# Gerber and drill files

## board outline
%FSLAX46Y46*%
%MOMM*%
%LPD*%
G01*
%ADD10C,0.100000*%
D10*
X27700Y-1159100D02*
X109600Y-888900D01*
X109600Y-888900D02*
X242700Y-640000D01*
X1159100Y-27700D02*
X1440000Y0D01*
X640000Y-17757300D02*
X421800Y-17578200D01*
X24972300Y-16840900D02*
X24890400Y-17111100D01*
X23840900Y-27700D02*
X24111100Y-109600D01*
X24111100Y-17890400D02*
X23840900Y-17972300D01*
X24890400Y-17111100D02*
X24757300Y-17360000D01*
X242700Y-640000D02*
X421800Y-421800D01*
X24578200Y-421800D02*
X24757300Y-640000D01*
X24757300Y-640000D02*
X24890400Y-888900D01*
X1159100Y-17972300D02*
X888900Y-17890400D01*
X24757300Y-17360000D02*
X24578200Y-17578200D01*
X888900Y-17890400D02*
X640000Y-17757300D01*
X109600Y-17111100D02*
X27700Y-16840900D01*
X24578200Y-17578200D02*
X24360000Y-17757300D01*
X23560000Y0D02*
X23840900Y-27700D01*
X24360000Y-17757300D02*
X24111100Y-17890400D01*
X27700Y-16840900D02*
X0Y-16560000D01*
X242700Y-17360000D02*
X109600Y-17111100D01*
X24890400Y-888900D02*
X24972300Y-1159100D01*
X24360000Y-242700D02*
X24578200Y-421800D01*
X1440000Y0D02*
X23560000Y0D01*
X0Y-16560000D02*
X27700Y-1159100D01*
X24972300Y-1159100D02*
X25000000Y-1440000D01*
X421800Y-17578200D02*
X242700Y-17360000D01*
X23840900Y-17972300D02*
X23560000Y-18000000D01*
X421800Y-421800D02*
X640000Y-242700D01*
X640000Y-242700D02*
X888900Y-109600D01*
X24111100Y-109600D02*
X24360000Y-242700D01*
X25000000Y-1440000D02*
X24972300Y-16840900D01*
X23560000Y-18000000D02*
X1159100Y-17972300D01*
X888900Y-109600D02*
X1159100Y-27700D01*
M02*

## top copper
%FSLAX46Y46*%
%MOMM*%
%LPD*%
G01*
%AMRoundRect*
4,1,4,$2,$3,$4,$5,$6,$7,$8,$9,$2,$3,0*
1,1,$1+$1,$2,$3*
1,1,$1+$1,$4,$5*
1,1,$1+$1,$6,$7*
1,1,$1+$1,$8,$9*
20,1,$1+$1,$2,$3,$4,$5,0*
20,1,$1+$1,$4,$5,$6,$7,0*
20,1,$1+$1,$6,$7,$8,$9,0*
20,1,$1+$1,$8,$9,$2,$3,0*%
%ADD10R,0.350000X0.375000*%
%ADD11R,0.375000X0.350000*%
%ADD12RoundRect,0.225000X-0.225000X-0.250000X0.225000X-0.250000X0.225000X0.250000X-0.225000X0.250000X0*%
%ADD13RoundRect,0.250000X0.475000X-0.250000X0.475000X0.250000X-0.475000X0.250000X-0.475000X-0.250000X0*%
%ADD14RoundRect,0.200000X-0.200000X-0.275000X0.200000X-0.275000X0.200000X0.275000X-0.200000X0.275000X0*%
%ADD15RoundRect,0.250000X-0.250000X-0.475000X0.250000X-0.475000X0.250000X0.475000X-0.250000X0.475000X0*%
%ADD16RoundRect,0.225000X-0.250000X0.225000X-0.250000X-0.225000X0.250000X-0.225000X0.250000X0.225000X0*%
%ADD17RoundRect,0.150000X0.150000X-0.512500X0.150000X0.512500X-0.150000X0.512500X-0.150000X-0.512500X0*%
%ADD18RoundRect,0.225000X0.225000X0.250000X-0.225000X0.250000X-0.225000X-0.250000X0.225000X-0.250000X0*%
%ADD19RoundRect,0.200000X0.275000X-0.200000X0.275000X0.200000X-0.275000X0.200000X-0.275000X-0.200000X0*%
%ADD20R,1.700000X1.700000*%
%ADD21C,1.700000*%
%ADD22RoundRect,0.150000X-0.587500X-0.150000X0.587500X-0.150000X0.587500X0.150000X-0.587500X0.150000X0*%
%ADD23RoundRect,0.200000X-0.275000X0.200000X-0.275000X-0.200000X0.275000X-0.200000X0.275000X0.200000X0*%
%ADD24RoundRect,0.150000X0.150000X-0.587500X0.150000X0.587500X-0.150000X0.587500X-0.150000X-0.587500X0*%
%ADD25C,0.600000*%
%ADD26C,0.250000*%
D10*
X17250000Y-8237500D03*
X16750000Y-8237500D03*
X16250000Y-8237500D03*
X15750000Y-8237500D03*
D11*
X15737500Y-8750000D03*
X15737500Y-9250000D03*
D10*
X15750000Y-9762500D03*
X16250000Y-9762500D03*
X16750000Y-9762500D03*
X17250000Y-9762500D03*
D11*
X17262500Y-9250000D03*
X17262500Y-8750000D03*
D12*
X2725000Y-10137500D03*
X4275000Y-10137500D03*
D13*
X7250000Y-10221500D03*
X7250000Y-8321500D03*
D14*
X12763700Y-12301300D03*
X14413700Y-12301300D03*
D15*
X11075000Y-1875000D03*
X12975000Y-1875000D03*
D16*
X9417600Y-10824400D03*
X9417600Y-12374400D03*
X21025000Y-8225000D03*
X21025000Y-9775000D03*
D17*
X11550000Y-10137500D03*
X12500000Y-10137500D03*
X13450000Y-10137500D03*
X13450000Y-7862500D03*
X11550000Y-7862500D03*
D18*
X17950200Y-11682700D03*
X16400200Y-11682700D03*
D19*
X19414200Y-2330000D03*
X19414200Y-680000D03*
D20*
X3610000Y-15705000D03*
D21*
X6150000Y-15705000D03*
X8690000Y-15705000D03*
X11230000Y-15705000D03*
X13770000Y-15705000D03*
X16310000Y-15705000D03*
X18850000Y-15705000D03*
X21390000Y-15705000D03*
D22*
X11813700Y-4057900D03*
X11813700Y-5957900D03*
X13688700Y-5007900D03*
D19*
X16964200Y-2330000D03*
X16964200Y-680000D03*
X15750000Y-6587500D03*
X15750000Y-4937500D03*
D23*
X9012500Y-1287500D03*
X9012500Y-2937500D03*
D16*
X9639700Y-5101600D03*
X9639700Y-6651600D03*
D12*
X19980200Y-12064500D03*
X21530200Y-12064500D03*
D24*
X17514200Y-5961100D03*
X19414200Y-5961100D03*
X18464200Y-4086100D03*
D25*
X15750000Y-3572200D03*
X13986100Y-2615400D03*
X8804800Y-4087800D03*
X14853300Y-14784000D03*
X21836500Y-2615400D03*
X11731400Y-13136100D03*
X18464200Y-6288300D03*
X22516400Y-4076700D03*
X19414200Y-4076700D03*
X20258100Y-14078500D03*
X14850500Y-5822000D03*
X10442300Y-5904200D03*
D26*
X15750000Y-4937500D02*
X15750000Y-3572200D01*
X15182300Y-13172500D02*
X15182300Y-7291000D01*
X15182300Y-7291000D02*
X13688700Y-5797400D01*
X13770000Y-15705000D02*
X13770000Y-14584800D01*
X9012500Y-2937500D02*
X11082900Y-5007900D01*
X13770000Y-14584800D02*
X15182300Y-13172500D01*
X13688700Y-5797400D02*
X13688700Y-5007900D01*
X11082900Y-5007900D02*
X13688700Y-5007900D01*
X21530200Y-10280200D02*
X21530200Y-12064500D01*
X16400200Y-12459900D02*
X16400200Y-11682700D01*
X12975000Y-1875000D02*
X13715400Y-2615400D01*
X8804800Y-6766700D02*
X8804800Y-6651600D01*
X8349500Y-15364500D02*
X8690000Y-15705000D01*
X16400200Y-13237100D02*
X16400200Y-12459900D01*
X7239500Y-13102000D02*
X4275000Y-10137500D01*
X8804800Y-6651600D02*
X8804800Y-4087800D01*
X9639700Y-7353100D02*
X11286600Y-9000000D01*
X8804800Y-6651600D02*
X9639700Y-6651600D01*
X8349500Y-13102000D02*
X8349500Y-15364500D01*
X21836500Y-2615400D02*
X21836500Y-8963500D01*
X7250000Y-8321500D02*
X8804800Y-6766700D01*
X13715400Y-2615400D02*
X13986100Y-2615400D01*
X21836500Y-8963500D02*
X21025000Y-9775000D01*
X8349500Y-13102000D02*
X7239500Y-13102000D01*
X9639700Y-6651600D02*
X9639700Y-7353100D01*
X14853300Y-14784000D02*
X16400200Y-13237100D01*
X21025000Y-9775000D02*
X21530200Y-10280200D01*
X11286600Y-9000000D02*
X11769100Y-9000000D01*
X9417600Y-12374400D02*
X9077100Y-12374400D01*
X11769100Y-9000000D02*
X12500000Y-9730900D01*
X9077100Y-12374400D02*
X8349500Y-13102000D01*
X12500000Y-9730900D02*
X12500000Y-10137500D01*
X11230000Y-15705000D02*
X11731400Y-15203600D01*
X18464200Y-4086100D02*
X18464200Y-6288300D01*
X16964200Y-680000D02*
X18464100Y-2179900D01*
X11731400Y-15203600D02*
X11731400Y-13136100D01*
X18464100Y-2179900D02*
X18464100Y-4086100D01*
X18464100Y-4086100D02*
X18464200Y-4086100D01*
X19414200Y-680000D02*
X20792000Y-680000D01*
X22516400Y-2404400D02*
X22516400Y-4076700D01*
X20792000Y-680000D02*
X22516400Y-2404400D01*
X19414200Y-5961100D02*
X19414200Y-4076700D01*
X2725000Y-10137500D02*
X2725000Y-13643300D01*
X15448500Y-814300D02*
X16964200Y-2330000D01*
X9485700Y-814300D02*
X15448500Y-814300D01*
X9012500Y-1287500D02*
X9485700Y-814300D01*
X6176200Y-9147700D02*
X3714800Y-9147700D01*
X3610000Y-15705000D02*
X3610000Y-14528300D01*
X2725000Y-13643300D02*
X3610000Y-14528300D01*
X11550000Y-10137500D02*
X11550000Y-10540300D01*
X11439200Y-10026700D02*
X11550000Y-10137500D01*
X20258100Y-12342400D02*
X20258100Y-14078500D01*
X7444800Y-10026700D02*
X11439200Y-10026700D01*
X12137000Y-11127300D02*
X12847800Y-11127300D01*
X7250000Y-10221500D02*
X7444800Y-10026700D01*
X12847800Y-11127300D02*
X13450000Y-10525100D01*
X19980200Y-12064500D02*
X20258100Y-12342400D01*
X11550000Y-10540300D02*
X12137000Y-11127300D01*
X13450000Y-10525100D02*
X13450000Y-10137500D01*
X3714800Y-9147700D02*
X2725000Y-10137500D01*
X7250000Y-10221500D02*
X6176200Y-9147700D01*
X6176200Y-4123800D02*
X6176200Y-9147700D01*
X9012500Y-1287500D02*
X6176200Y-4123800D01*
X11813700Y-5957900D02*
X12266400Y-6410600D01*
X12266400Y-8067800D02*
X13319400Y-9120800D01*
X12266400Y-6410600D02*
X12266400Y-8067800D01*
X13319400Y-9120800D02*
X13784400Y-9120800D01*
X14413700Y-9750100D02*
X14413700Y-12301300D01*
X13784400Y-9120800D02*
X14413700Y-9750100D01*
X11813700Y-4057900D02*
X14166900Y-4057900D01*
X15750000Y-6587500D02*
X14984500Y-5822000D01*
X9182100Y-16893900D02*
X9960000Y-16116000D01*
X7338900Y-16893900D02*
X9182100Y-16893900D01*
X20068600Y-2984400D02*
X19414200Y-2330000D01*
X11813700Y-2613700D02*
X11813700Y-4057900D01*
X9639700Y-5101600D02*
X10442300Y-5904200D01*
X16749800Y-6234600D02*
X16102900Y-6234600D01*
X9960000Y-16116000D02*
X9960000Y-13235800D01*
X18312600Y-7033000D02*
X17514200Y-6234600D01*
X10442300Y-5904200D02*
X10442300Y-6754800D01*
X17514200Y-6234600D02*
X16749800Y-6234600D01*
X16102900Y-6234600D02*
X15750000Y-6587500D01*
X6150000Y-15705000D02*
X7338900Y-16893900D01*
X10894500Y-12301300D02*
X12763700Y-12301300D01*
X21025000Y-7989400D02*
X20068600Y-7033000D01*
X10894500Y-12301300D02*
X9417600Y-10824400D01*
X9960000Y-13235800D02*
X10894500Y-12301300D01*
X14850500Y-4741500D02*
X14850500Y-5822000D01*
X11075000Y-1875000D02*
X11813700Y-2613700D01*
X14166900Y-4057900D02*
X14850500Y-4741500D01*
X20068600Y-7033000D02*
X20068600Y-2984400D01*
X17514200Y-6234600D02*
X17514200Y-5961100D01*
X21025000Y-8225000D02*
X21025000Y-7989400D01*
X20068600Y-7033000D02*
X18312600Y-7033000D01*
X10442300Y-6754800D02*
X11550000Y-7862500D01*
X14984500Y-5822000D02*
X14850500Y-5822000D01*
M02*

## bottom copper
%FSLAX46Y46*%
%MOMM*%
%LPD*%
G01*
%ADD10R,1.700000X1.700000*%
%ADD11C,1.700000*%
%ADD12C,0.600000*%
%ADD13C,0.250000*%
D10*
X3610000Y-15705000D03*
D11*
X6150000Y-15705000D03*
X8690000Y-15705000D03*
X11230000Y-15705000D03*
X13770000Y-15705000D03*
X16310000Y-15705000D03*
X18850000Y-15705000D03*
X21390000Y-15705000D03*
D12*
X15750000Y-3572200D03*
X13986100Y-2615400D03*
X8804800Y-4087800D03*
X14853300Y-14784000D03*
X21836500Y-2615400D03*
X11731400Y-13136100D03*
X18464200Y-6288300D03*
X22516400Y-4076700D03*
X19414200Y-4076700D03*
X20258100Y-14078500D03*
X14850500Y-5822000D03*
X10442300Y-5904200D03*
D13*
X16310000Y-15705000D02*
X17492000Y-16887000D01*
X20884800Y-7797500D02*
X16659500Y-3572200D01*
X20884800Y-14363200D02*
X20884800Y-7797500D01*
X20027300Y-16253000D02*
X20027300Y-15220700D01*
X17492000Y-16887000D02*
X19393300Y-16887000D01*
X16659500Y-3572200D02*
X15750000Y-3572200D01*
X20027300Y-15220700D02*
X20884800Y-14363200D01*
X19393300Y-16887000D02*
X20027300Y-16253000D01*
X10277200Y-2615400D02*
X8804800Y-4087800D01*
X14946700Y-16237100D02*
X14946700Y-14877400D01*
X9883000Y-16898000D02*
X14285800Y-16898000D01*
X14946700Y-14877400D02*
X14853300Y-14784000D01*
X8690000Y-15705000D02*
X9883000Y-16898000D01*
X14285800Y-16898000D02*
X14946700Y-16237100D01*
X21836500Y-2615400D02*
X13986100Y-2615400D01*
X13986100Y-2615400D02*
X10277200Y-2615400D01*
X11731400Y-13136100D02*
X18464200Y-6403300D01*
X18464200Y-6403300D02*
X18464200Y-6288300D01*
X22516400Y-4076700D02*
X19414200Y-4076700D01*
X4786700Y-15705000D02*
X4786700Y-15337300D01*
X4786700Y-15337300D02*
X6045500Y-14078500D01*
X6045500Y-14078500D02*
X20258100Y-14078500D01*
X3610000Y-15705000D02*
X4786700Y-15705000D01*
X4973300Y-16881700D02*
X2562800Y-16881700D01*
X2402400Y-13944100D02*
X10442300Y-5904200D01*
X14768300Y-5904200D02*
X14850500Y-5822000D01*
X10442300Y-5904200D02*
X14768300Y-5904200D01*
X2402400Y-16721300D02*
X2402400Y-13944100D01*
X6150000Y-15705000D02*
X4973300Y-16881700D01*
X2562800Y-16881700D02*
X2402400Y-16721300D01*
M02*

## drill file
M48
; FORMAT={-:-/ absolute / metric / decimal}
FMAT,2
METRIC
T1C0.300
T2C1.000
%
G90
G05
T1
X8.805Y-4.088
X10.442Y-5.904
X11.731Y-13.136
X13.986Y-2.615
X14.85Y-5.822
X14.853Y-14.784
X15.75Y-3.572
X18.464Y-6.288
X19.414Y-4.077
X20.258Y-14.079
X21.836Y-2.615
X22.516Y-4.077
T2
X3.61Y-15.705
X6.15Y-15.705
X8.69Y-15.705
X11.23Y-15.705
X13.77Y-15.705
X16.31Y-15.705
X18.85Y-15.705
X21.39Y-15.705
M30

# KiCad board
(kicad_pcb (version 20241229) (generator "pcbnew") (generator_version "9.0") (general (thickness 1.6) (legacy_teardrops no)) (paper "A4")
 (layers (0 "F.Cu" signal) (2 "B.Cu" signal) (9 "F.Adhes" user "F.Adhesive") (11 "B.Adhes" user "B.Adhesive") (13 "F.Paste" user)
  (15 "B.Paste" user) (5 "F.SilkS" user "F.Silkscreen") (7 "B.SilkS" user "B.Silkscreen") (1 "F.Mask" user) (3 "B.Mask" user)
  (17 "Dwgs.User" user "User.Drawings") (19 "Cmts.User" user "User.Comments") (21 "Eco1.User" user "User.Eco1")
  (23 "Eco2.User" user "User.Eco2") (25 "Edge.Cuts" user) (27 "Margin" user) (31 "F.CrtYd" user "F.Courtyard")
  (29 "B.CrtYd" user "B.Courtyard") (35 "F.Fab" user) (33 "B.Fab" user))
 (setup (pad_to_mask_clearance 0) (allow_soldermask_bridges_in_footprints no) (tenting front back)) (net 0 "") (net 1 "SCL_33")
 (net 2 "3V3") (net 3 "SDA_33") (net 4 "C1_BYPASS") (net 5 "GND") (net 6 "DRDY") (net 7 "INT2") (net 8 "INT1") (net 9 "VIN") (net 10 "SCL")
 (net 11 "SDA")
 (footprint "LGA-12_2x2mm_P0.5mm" (layer "F.Cu") (at 16.5 9 -90)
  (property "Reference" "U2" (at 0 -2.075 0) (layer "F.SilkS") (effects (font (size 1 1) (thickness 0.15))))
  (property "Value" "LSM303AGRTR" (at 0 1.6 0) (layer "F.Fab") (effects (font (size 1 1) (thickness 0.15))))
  (pad "1" smd rect (at -0.7625 -0.75 270) (size 0.375 0.35) (layers "F.Cu" "F.Mask" "F.Paste") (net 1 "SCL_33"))
  (pad "2" smd rect (at -0.7625 -0.25 270) (size 0.375 0.35) (layers "F.Cu" "F.Mask" "F.Paste") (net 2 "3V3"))
  (pad "3" smd rect (at -0.7625 0.25 270) (size 0.375 0.35) (layers "F.Cu" "F.Mask" "F.Paste") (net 2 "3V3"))
  (pad "4" smd rect (at -0.7625 0.75 270) (size 0.375 0.35) (layers "F.Cu" "F.Mask" "F.Paste") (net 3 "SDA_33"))
  (pad "5" smd rect (at -0.25 0.7625) (size 0.375 0.35) (layers "F.Cu" "F.Mask" "F.Paste") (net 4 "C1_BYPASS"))
  (pad "6" smd rect (at 0.25 0.7625) (size 0.375 0.35) (layers "F.Cu" "F.Mask" "F.Paste") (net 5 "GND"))
  (pad "7" smd rect (at 0.7625 0.75 270) (size 0.375 0.35) (layers "F.Cu" "F.Mask" "F.Paste") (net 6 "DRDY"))
  (pad "8" smd rect (at 0.7625 0.25 270) (size 0.375 0.35) (layers "F.Cu" "F.Mask" "F.Paste") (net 5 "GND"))
  (pad "9" smd rect (at 0.7625 -0.25 270) (size 0.375 0.35) (layers "F.Cu" "F.Mask" "F.Paste") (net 2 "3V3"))
  (pad "10" smd rect (at 0.7625 -0.75 270) (size 0.375 0.35) (layers "F.Cu" "F.Mask" "F.Paste") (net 2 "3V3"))
  (pad "11" smd rect (at 0.25 -0.7625) (size 0.375 0.35) (layers "F.Cu" "F.Mask" "F.Paste") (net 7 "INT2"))
  (pad "12" smd rect (at -0.25 -0.7625) (size 0.375 0.35) (layers "F.Cu" "F.Mask" "F.Paste") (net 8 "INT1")))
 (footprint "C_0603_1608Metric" (layer "F.Cu") (at 3.5 10.1375)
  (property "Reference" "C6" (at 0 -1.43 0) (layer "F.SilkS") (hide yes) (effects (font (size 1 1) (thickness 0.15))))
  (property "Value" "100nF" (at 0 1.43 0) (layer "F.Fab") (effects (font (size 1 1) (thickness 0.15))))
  (pad "1" smd roundrect (at -0.775 0) (size 0.9 0.95) (layers "F.Cu" "F.Mask" "F.Paste") (roundrect_rratio 0.25) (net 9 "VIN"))
  (pad "2" smd roundrect (at 0.775 0) (size 0.9 0.95) (layers "F.Cu" "F.Mask" "F.Paste") (roundrect_rratio 0.25) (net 5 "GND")))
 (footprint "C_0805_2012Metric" (layer "F.Cu") (at 7.25 9.2715 90)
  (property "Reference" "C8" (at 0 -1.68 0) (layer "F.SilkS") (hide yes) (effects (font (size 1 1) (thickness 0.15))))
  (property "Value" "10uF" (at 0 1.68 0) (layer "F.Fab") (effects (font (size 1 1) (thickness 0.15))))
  (pad "1" smd roundrect (at -0.95 0 90) (size 1 1.45) (layers "F.Cu" "F.Mask" "F.Paste") (roundrect_rratio 0.25) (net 9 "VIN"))
  (pad "2" smd roundrect (at 0.95 0 90) (size 1 1.45) (layers "F.Cu" "F.Mask" "F.Paste") (roundrect_rratio 0.25) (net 5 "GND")))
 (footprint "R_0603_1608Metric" (layer "F.Cu") (at 13.5887 12.3013)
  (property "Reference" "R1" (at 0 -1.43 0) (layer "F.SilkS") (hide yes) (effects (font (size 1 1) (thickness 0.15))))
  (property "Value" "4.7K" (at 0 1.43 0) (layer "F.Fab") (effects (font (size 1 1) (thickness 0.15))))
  (pad "1" smd roundrect (at -0.825 0) (size 0.8 0.95) (layers "F.Cu" "F.Mask" "F.Paste") (roundrect_rratio 0.25) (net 2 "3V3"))
  (pad "2" smd roundrect (at 0.825 0) (size 0.8 0.95) (layers "F.Cu" "F.Mask" "F.Paste") (roundrect_rratio 0.25) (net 3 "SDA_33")))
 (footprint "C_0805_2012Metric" (layer "F.Cu") (at 12.025 1.875)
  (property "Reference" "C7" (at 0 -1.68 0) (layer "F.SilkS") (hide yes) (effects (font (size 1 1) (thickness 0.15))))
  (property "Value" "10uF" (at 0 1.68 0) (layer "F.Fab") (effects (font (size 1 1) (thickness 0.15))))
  (pad "1" smd roundrect (at -0.95 0) (size 1 1.45) (layers "F.Cu" "F.Mask" "F.Paste") (roundrect_rratio 0.25) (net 2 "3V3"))
  (pad "2" smd roundrect (at 0.95 0) (size 1 1.45) (layers "F.Cu" "F.Mask" "F.Paste") (roundrect_rratio 0.25) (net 5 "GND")))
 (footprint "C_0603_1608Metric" (layer "F.Cu") (at 9.4176 11.5994 -90)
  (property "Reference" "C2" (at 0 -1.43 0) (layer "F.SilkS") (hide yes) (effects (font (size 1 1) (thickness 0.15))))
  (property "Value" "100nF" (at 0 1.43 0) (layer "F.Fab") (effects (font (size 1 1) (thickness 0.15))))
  (pad "1" smd roundrect (at -0.775 0 270) (size 0.9 0.95) (layers "F.Cu" "F.Mask" "F.Paste") (roundrect_rratio 0.25) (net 2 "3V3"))
  (pad "2" smd roundrect (at 0.775 0 270) (size 0.9 0.95) (layers "F.Cu" "F.Mask" "F.Paste") (roundrect_rratio 0.25) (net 5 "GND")))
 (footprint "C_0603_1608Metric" (layer "F.Cu") (at 21.025 9 -90)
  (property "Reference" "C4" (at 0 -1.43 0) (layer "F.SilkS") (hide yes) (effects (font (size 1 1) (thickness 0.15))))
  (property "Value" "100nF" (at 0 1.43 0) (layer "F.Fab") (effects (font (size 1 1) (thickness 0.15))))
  (pad "1" smd roundrect (at -0.775 0 270) (size 0.9 0.95) (layers "F.Cu" "F.Mask" "F.Paste") (roundrect_rratio 0.25) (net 2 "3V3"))
  (pad "2" smd roundrect (at 0.775 0 270) (size 0.9 0.95) (layers "F.Cu" "F.Mask" "F.Paste") (roundrect_rratio 0.25) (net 5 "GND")))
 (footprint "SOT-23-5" (layer "F.Cu") (at 12.5 9 90)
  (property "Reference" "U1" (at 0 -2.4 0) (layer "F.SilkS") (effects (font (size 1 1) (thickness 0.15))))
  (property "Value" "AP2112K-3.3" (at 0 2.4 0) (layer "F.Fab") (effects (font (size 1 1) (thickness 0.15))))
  (pad "1" smd roundrect (at -1.1375 -0.95 90) (size 1.325 0.6) (layers "F.Cu" "F.Mask" "F.Paste") (roundrect_rratio 0.25) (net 9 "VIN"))
  (pad "2" smd roundrect (at -1.1375 0 90) (size 1.325 0.6) (layers "F.Cu" "F.Mask" "F.Paste") (roundrect_rratio 0.25) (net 5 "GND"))
  (pad "3" smd roundrect (at -1.1375 0.95 90) (size 1.325 0.6) (layers "F.Cu" "F.Mask" "F.Paste") (roundrect_rratio 0.25) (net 9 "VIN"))
  (pad "4" smd roundrect (at 1.1375 0.95 90) (size 1.325 0.6) (layers "F.Cu" "F.Mask" "F.Paste") (roundrect_rratio 0.25))
  (pad "5" smd roundrect (at 1.1375 -0.95 90) (size 1.325 0.6) (layers "F.Cu" "F.Mask" "F.Paste") (roundrect_rratio 0.25) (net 2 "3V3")))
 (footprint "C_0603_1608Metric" (layer "F.Cu") (at 17.1752 11.6827 180)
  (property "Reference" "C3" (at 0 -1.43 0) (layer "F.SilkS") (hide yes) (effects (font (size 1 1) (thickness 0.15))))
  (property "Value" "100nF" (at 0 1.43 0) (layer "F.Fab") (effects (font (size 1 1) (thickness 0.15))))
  (pad "1" smd roundrect (at -0.775 0 180) (size 0.9 0.95) (layers "F.Cu" "F.Mask" "F.Paste") (roundrect_rratio 0.25) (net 4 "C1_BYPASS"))
  (pad "2" smd roundrect (at 0.775 0 180) (size 0.9 0.95) (layers "F.Cu" "F.Mask" "F.Paste") (roundrect_rratio 0.25) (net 5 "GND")))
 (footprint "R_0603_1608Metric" (layer "F.Cu") (at 19.4142 1.505 90)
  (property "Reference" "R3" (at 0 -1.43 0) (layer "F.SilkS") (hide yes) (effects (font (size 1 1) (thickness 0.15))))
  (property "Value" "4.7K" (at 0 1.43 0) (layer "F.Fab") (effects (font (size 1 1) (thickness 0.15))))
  (pad "1" smd roundrect (at -0.825 0 90) (size 0.8 0.95) (layers "F.Cu" "F.Mask" "F.Paste") (roundrect_rratio 0.25) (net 2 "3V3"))
  (pad "2" smd roundrect (at 0.825 0 90) (size 0.8 0.95) (layers "F.Cu" "F.Mask" "F.Paste") (roundrect_rratio 0.25) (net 1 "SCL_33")))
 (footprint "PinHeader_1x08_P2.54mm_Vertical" (layer "F.Cu") (at 3.61 15.705 90)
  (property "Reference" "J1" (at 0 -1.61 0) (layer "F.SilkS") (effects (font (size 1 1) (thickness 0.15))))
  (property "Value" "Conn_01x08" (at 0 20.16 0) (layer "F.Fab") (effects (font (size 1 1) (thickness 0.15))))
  (pad "1" thru_hole rect (at 0 0 90) (size 1.7 1.7) (drill 1) (layers "*.Cu" "*.Mask") (remove_unused_layers no) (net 9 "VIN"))
  (pad "2" thru_hole circle (at 0 2.54 90) (size 1.7 1.7) (drill 1) (layers "*.Cu" "*.Mask") (remove_unused_layers no) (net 2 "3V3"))
  (pad "3" thru_hole circle (at 0 5.08 90) (size 1.7 1.7) (drill 1) (layers "*.Cu" "*.Mask") (remove_unused_layers no) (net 5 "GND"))
  (pad "4" thru_hole circle (at 0 7.62 90) (size 1.7 1.7) (drill 1) (layers "*.Cu" "*.Mask") (remove_unused_layers no) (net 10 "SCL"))
  (pad "5" thru_hole circle (at 0 10.16 90) (size 1.7 1.7) (drill 1) (layers "*.Cu" "*.Mask") (remove_unused_layers no) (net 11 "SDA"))
  (pad "6" thru_hole circle (at 0 12.7 90) (size 1.7 1.7) (drill 1) (layers "*.Cu" "*.Mask") (remove_unused_layers no) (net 6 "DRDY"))
  (pad "7" thru_hole circle (at 0 15.24 90) (size 1.7 1.7) (drill 1) (layers "*.Cu" "*.Mask") (remove_unused_layers no) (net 8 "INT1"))
  (pad "8" thru_hole circle (at 0 17.78 90) (size 1.7 1.7) (drill 1) (layers "*.Cu" "*.Mask") (remove_unused_layers no) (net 7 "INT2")))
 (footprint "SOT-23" (layer "F.Cu") (at 12.7512 5.0079)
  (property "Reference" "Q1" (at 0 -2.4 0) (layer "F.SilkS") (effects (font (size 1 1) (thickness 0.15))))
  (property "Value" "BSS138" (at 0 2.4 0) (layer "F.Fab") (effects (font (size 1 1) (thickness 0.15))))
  (pad "1" smd roundrect (at -0.9375 -0.95) (size 1.475 0.6) (layers "F.Cu" "F.Mask" "F.Paste") (roundrect_rratio 0.25) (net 2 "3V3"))
  (pad "2" smd roundrect (at -0.9375 0.95) (size 1.475 0.6) (layers "F.Cu" "F.Mask" "F.Paste") (roundrect_rratio 0.25) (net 3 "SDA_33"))
  (pad "3" smd roundrect (at 0.9375 0) (size 1.475 0.6) (layers "F.Cu" "F.Mask" "F.Paste") (roundrect_rratio 0.25) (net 11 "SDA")))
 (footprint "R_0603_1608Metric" (layer "F.Cu") (at 16.9642 1.505 90)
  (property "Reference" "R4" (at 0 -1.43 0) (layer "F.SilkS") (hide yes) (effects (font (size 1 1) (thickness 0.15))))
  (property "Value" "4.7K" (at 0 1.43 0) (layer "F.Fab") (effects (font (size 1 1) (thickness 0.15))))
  (pad "1" smd roundrect (at -0.825 0 90) (size 0.8 0.95) (layers "F.Cu" "F.Mask" "F.Paste") (roundrect_rratio 0.25) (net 9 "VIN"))
  (pad "2" smd roundrect (at 0.825 0 90) (size 0.8 0.95) (layers "F.Cu" "F.Mask" "F.Paste") (roundrect_rratio 0.25) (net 10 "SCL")))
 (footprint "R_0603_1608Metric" (layer "F.Cu") (at 15.75 5.7625 90)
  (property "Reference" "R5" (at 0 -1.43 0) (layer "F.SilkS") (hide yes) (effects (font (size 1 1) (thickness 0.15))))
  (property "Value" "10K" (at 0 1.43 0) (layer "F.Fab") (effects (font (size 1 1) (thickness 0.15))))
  (pad "1" smd roundrect (at -0.825 0 90) (size 0.8 0.95) (layers "F.Cu" "F.Mask" "F.Paste") (roundrect_rratio 0.25) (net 2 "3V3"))
  (pad "2" smd roundrect (at 0.825 0 90) (size 0.8 0.95) (layers "F.Cu" "F.Mask" "F.Paste") (roundrect_rratio 0.25) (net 6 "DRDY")))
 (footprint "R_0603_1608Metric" (layer "F.Cu") (at 9.0125 2.1125 -90)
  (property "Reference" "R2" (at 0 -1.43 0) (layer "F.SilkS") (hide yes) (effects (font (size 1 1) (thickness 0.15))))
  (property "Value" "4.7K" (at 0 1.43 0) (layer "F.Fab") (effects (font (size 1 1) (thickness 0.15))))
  (pad "1" smd roundrect (at -0.825 0 270) (size 0.8 0.95) (layers "F.Cu" "F.Mask" "F.Paste") (roundrect_rratio 0.25) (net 9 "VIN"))
  (pad "2" smd roundrect (at 0.825 0 270) (size 0.8 0.95) (layers "F.Cu" "F.Mask" "F.Paste") (roundrect_rratio 0.25) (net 11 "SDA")))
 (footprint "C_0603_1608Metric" (layer "F.Cu") (at 9.6397 5.8766 -90)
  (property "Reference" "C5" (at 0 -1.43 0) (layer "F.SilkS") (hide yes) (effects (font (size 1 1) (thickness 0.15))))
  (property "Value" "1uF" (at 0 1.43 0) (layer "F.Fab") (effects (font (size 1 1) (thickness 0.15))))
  (pad "1" smd roundrect (at -0.775 0 270) (size 0.9 0.95) (layers "F.Cu" "F.Mask" "F.Paste") (roundrect_rratio 0.25) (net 2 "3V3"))
  (pad "2" smd roundrect (at 0.775 0 270) (size 0.9 0.95) (layers "F.Cu" "F.Mask" "F.Paste") (roundrect_rratio 0.25) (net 5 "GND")))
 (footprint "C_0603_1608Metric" (layer "F.Cu") (at 20.7552 12.0645)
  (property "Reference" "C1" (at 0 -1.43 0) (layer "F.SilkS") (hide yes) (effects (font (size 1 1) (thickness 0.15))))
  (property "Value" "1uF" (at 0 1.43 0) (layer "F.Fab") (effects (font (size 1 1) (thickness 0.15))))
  (pad "1" smd roundrect (at -0.775 0) (size 0.9 0.95) (layers "F.Cu" "F.Mask" "F.Paste") (roundrect_rratio 0.25) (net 9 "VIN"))
  (pad "2" smd roundrect (at 0.775 0) (size 0.9 0.95) (layers "F.Cu" "F.Mask" "F.Paste") (roundrect_rratio 0.25) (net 5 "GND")))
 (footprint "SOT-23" (layer "F.Cu") (at 18.4642 5.0236 90)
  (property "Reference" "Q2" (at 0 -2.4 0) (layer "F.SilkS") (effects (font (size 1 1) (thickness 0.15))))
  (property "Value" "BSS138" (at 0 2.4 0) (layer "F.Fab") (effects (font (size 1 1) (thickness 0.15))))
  (pad "1" smd roundrect (at -0.9375 -0.95 90) (size 1.475 0.6) (layers "F.Cu" "F.Mask" "F.Paste") (roundrect_rratio 0.25) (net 2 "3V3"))
  (pad "2" smd roundrect (at -0.9375 0.95 90) (size 1.475 0.6) (layers "F.Cu" "F.Mask" "F.Paste") (roundrect_rratio 0.25) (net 1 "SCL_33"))
  (pad "3" smd roundrect (at 0.9375 0 90) (size 1.475 0.6) (layers "F.Cu" "F.Mask" "F.Paste") (roundrect_rratio 0.25) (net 10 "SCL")))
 (gr_line (start 0.0277 1.1591) (end 0.1096 0.8889) (stroke (width 0.1) (type solid)) (layer "Edge.Cuts"))
 (gr_line (start 0.1096 0.8889) (end 0.2427 0.64) (stroke (width 0.1) (type solid)) (layer "Edge.Cuts"))
 (gr_line (start 1.1591 0.0277) (end 1.44 0) (stroke (width 0.1) (type solid)) (layer "Edge.Cuts"))
 (gr_line (start 0.64 17.7573) (end 0.4218 17.5782) (stroke (width 0.1) (type solid)) (layer "Edge.Cuts"))
 (gr_line (start 24.9723 16.8409) (end 24.8904 17.1111) (stroke (width 0.1) (type solid)) (layer "Edge.Cuts"))
 (gr_line (start 23.8409 0.0277) (end 24.1111 0.1096) (stroke (width 0.1) (type solid)) (layer "Edge.Cuts"))
 (gr_line (start 24.1111 17.8904) (end 23.8409 17.9723) (stroke (width 0.1) (type solid)) (layer "Edge.Cuts"))
 (gr_line (start 24.8904 17.1111) (end 24.7573 17.36) (stroke (width 0.1) (type solid)) (layer "Edge.Cuts"))
 (gr_line (start 0.2427 0.64) (end 0.4218 0.4218) (stroke (width 0.1) (type solid)) (layer "Edge.Cuts"))
 (gr_line (start 24.5782 0.4218) (end 24.7573 0.64) (stroke (width 0.1) (type solid)) (layer "Edge.Cuts"))
 (gr_line (start 24.7573 0.64) (end 24.8904 0.8889) (stroke (width 0.1) (type solid)) (layer "Edge.Cuts"))
 (gr_line (start 1.1591 17.9723) (end 0.8889 17.8904) (stroke (width 0.1) (type solid)) (layer "Edge.Cuts"))
 (gr_line (start 24.7573 17.36) (end 24.5782 17.5782) (stroke (width 0.1) (type solid)) (layer "Edge.Cuts"))
 (gr_line (start 0.8889 17.8904) (end 0.64 17.7573) (stroke (width 0.1) (type solid)) (layer "Edge.Cuts"))
 (gr_line (start 0.1096 17.1111) (end 0.0277 16.8409) (stroke (width 0.1) (type solid)) (layer "Edge.Cuts"))
 (gr_line (start 24.5782 17.5782) (end 24.36 17.7573) (stroke (width 0.1) (type solid)) (layer "Edge.Cuts"))
 (gr_line (start 23.56 0) (end 23.8409 0.0277) (stroke (width 0.1) (type solid)) (layer "Edge.Cuts"))
 (gr_line (start 24.36 17.7573) (end 24.1111 17.8904) (stroke (width 0.1) (type solid)) (layer "Edge.Cuts"))
 (gr_line (start 0.0277 16.8409) (end 0 16.56) (stroke (width 0.1) (type solid)) (layer "Edge.Cuts"))
 (gr_line (start 0.2427 17.36) (end 0.1096 17.1111) (stroke (width 0.1) (type solid)) (layer "Edge.Cuts"))
 (gr_line (start 24.8904 0.8889) (end 24.9723 1.1591) (stroke (width 0.1) (type solid)) (layer "Edge.Cuts"))
 (gr_line (start 24.36 0.2427) (end 24.5782 0.4218) (stroke (width 0.1) (type solid)) (layer "Edge.Cuts"))
 (gr_line (start 1.44 0) (end 23.56 0) (stroke (width 0.1) (type solid)) (layer "Edge.Cuts"))
 (gr_line (start 0 16.56) (end 0.0277 1.1591) (stroke (width 0.1) (type solid)) (layer "Edge.Cuts"))
 (gr_line (start 24.9723 1.1591) (end 25 1.44) (stroke (width 0.1) (type solid)) (layer "Edge.Cuts"))
 (gr_line (start 0.4218 17.5782) (end 0.2427 17.36) (stroke (width 0.1) (type solid)) (layer "Edge.Cuts"))
 (gr_line (start 23.8409 17.9723) (end 23.56 18) (stroke (width 0.1) (type solid)) (layer "Edge.Cuts"))
 (gr_line (start 0.4218 0.4218) (end 0.64 0.2427) (stroke (width 0.1) (type solid)) (layer "Edge.Cuts"))
 (gr_line (start 0.64 0.2427) (end 0.8889 0.1096) (stroke (width 0.1) (type solid)) (layer "Edge.Cuts"))
 (gr_line (start 24.1111 0.1096) (end 24.36 0.2427) (stroke (width 0.1) (type solid)) (layer "Edge.Cuts"))
 (gr_line (start 25 1.44) (end 24.9723 16.8409) (stroke (width 0.1) (type solid)) (layer "Edge.Cuts"))
 (gr_line (start 23.56 18) (end 1.1591 17.9723) (stroke (width 0.1) (type solid)) (layer "Edge.Cuts"))
 (gr_line (start 0.8889 0.1096) (end 1.1591 0.0277) (stroke (width 0.1) (type solid)) (layer "Edge.Cuts"))
 (segment (start 15.75 4.9375) (end 15.75 3.5722) (width 0.25) (layer "F.Cu") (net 6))
 (via (at 15.75 3.5722) (size 0.6) (drill 0.3) (layers "F.Cu" "B.Cu") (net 6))
 (segment (start 16.31 15.705) (end 17.492 16.887) (width 0.25) (layer "B.Cu") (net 6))
 (segment (start 20.8848 7.7975) (end 16.6595 3.5722) (width 0.25) (layer "B.Cu") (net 6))
 (segment (start 20.8848 14.3632) (end 20.8848 7.7975) (width 0.25) (layer "B.Cu") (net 6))
 (segment (start 20.0273 16.253) (end 20.0273 15.2207) (width 0.25) (layer "B.Cu") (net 6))
 (segment (start 17.492 16.887) (end 19.3933 16.887) (width 0.25) (layer "B.Cu") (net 6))
 (segment (start 16.6595 3.5722) (end 15.75 3.5722) (width 0.25) (layer "B.Cu") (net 6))
 (segment (start 20.0273 15.2207) (end 20.8848 14.3632) (width 0.25) (layer "B.Cu") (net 6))
 (segment (start 19.3933 16.887) (end 20.0273 16.253) (width 0.25) (layer "B.Cu") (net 6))
 (segment (start 15.1823 13.1725) (end 15.1823 7.291) (width 0.25) (layer "F.Cu") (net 11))
 (segment (start 15.1823 7.291) (end 13.6887 5.7974) (width 0.25) (layer "F.Cu") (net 11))
 (segment (start 13.77 15.705) (end 13.77 14.5848) (width 0.25) (layer "F.Cu") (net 11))
 (segment (start 9.0125 2.9375) (end 11.0829 5.0079) (width 0.25) (layer "F.Cu") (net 11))
 (segment (start 13.77 14.5848) (end 15.1823 13.1725) (width 0.25) (layer "F.Cu") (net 11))
 (segment (start 13.6887 5.7974) (end 13.6887 5.0079) (width 0.25) (layer "F.Cu") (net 11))
 (segment (start 11.0829 5.0079) (end 13.6887 5.0079) (width 0.25) (layer "F.Cu") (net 11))
 (segment (start 21.5302 10.2802) (end 21.5302 12.0645) (width 0.25) (layer "F.Cu") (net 5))
 (segment (start 16.4002 12.4599) (end 16.4002 11.6827) (width 0.25) (layer "F.Cu") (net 5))
 (segment (start 12.975 1.875) (end 13.7154 2.6154) (width 0.25) (layer "F.Cu") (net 5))
 (segment (start 8.8048 6.7667) (end 8.8048 6.6516) (width 0.25) (layer "F.Cu") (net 5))
 (segment (start 8.3495 15.3645) (end 8.69 15.705) (width 0.25) (layer "F.Cu") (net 5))
 (segment (start 16.4002 13.2371) (end 16.4002 12.4599) (width 0.25) (layer "F.Cu") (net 5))
 (segment (start 7.2395 13.102) (end 4.275 10.1375) (width 0.25) (layer "F.Cu") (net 5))
 (segment (start 8.8048 6.6516) (end 8.8048 4.0878) (width 0.25) (layer "F.Cu") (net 5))
 (segment (start 9.6397 7.3531) (end 11.2866 9) (width 0.25) (layer "F.Cu") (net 5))
 (segment (start 8.8048 6.6516) (end 9.6397 6.6516) (width 0.25) (layer "F.Cu") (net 5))
 (segment (start 8.3495 13.102) (end 8.3495 15.3645) (width 0.25) (layer "F.Cu") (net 5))
 (segment (start 21.8365 2.6154) (end 21.8365 8.9635) (width 0.25) (layer "F.Cu") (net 5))
 (segment (start 7.25 8.3215) (end 8.8048 6.7667) (width 0.25) (layer "F.Cu") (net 5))
 (segment (start 13.7154 2.6154) (end 13.9861 2.6154) (width 0.25) (layer "F.Cu") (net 5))
 (segment (start 21.8365 8.9635) (end 21.025 9.775) (width 0.25) (layer "F.Cu") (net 5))
 (segment (start 8.3495 13.102) (end 7.2395 13.102) (width 0.25) (layer "F.Cu") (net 5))
 (segment (start 9.6397 6.6516) (end 9.6397 7.3531) (width 0.25) (layer "F.Cu") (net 5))
 (segment (start 14.8533 14.784) (end 16.4002 13.2371) (width 0.25) (layer "F.Cu") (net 5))
 (segment (start 21.025 9.775) (end 21.5302 10.2802) (width 0.25) (layer "F.Cu") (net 5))
 (segment (start 11.2866 9) (end 11.7691 9) (width 0.25) (layer "F.Cu") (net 5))
 (segment (start 9.4176 12.3744) (end 9.0771 12.3744) (width 0.25) (layer "F.Cu") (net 5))
 (segment (start 11.7691 9) (end 12.5 9.7309) (width 0.25) (layer "F.Cu") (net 5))
 (segment (start 9.0771 12.3744) (end 8.3495 13.102) (width 0.25) (layer "F.Cu") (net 5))
 (segment (start 12.5 9.7309) (end 12.5 10.1375) (width 0.25) (layer "F.Cu") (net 5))
 (via (at 13.9861 2.6154) (size 0.6) (drill 0.3) (layers "F.Cu" "B.Cu") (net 5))
 (via (at 8.8048 4.0878) (size 0.6) (drill 0.3) (layers "F.Cu" "B.Cu") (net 5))
 (via (at 14.8533 14.784) (size 0.6) (drill 0.3) (layers "F.Cu" "B.Cu") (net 5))
 (via (at 21.8365 2.6154) (size 0.6) (drill 0.3) (layers "F.Cu" "B.Cu") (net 5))
 (segment (start 10.2772 2.6154) (end 8.8048 4.0878) (width 0.25) (layer "B.Cu") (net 5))
 (segment (start 14.9467 16.2371) (end 14.9467 14.8774) (width 0.25) (layer "B.Cu") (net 5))
 (segment (start 9.883 16.898) (end 14.2858 16.898) (width 0.25) (layer "B.Cu") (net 5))
 (segment (start 14.9467 14.8774) (end 14.8533 14.784) (width 0.25) (layer "B.Cu") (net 5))
 (segment (start 8.69 15.705) (end 9.883 16.898) (width 0.25) (layer "B.Cu") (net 5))
 (segment (start 14.2858 16.898) (end 14.9467 16.2371) (width 0.25) (layer "B.Cu") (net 5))
 (segment (start 21.8365 2.6154) (end 13.9861 2.6154) (width 0.25) (layer "B.Cu") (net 5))
 (segment (start 13.9861 2.6154) (end 10.2772 2.6154) (width 0.25) (layer "B.Cu") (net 5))
 (segment (start 11.23 15.705) (end 11.7314 15.2036) (width 0.25) (layer "F.Cu") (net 10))
 (segment (start 18.4642 4.0861) (end 18.4642 6.2883) (width 0.25) (layer "F.Cu") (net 10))
 (segment (start 16.9642 0.68) (end 18.4641 2.1799) (width 0.25) (layer "F.Cu") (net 10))
 (segment (start 11.7314 15.2036) (end 11.7314 13.1361) (width 0.25) (layer "F.Cu") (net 10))
 (segment (start 18.4641 2.1799) (end 18.4641 4.0861) (width 0.25) (layer "F.Cu") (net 10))
 (segment (start 18.4641 4.0861) (end 18.4642 4.0861) (width 0.25) (layer "F.Cu") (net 10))
 (via (at 11.7314 13.1361) (size 0.6) (drill 0.3) (layers "F.Cu" "B.Cu") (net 10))
 (via (at 18.4642 6.2883) (size 0.6) (drill 0.3) (layers "F.Cu" "B.Cu") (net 10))
 (segment (start 11.7314 13.1361) (end 18.4642 6.4033) (width 0.25) (layer "B.Cu") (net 10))
 (segment (start 18.4642 6.4033) (end 18.4642 6.2883) (width 0.25) (layer "B.Cu") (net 10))
 (segment (start 19.4142 0.68) (end 20.792 0.68) (width 0.25) (layer "F.Cu") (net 1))
 (segment (start 22.5164 2.4044) (end 22.5164 4.0767) (width 0.25) (layer "F.Cu") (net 1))
 (segment (start 20.792 0.68) (end 22.5164 2.4044) (width 0.25) (layer "F.Cu") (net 1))
 (segment (start 19.4142 5.9611) (end 19.4142 4.0767) (width 0.25) (layer "F.Cu") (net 1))
 (via (at 22.5164 4.0767) (size 0.6) (drill 0.3) (layers "F.Cu" "B.Cu") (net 1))
 (via (at 19.4142 4.0767) (size 0.6) (drill 0.3) (layers "F.Cu" "B.Cu") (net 1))
 (segment (start 22.5164 4.0767) (end 19.4142 4.0767) (width 0.25) (layer "B.Cu") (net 1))
 (segment (start 2.725 10.1375) (end 2.725 13.6433) (width 0.25) (layer "F.Cu") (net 9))
 (segment (start 15.4485 0.8143) (end 16.9642 2.33) (width 0.25) (layer "F.Cu") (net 9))
 (segment (start 9.4857 0.8143) (end 15.4485 0.8143) (width 0.25) (layer "F.Cu") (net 9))
 (segment (start 9.0125 1.2875) (end 9.4857 0.8143) (width 0.25) (layer "F.Cu") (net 9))
 (segment (start 6.1762 9.1477) (end 3.7148 9.1477) (width 0.25) (layer "F.Cu") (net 9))
 (segment (start 3.61 15.705) (end 3.61 14.5283) (width 0.25) (layer "F.Cu") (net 9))
 (segment (start 2.725 13.6433) (end 3.61 14.5283) (width 0.25) (layer "F.Cu") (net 9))
 (segment (start 11.55 10.1375) (end 11.55 10.5403) (width 0.25) (layer "F.Cu") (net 9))
 (segment (start 11.4392 10.0267) (end 11.55 10.1375) (width 0.25) (layer "F.Cu") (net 9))
 (segment (start 20.2581 12.3424) (end 20.2581 14.0785) (width 0.25) (layer "F.Cu") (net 9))
 (segment (start 7.4448 10.0267) (end 11.4392 10.0267) (width 0.25) (layer "F.Cu") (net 9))
 (segment (start 12.137 11.1273) (end 12.8478 11.1273) (width 0.25) (layer "F.Cu") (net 9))
 (segment (start 7.25 10.2215) (end 7.4448 10.0267) (width 0.25) (layer "F.Cu") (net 9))
 (segment (start 12.8478 11.1273) (end 13.45 10.5251) (width 0.25) (layer "F.Cu") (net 9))
 (segment (start 19.9802 12.0645) (end 20.2581 12.3424) (width 0.25) (layer "F.Cu") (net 9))
 (segment (start 11.55 10.5403) (end 12.137 11.1273) (width 0.25) (layer "F.Cu") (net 9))
 (segment (start 13.45 10.5251) (end 13.45 10.1375) (width 0.25) (layer "F.Cu") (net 9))
 (segment (start 3.7148 9.1477) (end 2.725 10.1375) (width 0.25) (layer "F.Cu") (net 9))
 (segment (start 7.25 10.2215) (end 6.1762 9.1477) (width 0.25) (layer "F.Cu") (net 9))
 (segment (start 6.1762 4.1238) (end 6.1762 9.1477) (width 0.25) (layer "F.Cu") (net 9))
 (segment (start 9.0125 1.2875) (end 6.1762 4.1238) (width 0.25) (layer "F.Cu") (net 9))
 (via (at 20.2581 14.0785) (size 0.6) (drill 0.3) (layers "F.Cu" "B.Cu") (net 9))
 (segment (start 4.7867 15.705) (end 4.7867 15.3373) (width 0.25) (layer "B.Cu") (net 9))
 (segment (start 4.7867 15.3373) (end 6.0455 14.0785) (width 0.25) (layer "B.Cu") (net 9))
 (segment (start 6.0455 14.0785) (end 20.2581 14.0785) (width 0.25) (layer "B.Cu") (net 9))
 (segment (start 3.61 15.705) (end 4.7867 15.705) (width 0.25) (layer "B.Cu") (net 9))
 (segment (start 11.8137 5.9579) (end 12.2664 6.4106) (width 0.25) (layer "F.Cu") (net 3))
 (segment (start 12.2664 8.0678) (end 13.3194 9.1208) (width 0.25) (layer "F.Cu") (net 3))
 (segment (start 12.2664 6.4106) (end 12.2664 8.0678) (width 0.25) (layer "F.Cu") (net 3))
 (segment (start 13.3194 9.1208) (end 13.7844 9.1208) (width 0.25) (layer "F.Cu") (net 3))
 (segment (start 14.4137 9.7501) (end 14.4137 12.3013) (width 0.25) (layer "F.Cu") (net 3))
 (segment (start 13.7844 9.1208) (end 14.4137 9.7501) (width 0.25) (layer "F.Cu") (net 3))
 (segment (start 11.8137 4.0579) (end 14.1669 4.0579) (width 0.25) (layer "F.Cu") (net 2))
 (segment (start 15.75 6.5875) (end 14.9845 5.822) (width 0.25) (layer "F.Cu") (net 2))
 (segment (start 9.1821 16.8939) (end 9.96 16.116) (width 0.25) (layer "F.Cu") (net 2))
 (segment (start 7.3389 16.8939) (end 9.1821 16.8939) (width 0.25) (layer "F.Cu") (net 2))
 (segment (start 20.0686 2.9844) (end 19.4142 2.33) (width 0.25) (layer "F.Cu") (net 2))
 (segment (start 11.8137 2.6137) (end 11.8137 4.0579) (width 0.25) (layer "F.Cu") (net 2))
 (segment (start 9.6397 5.1016) (end 10.4423 5.9042) (width 0.25) (layer "F.Cu") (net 2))
 (segment (start 16.7498 6.2346) (end 16.1029 6.2346) (width 0.25) (layer "F.Cu") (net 2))
 (segment (start 9.96 16.116) (end 9.96 13.2358) (width 0.25) (layer "F.Cu") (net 2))
 (segment (start 18.3126 7.033) (end 17.5142 6.2346) (width 0.25) (layer "F.Cu") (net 2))
 (segment (start 10.4423 5.9042) (end 10.4423 6.7548) (width 0.25) (layer "F.Cu") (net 2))
 (segment (start 17.5142 6.2346) (end 16.7498 6.2346) (width 0.25) (layer "F.Cu") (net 2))
 (segment (start 16.1029 6.2346) (end 15.75 6.5875) (width 0.25) (layer "F.Cu") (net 2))
 (segment (start 6.15 15.705) (end 7.3389 16.8939) (width 0.25) (layer "F.Cu") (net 2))
 (segment (start 10.8945 12.3013) (end 12.7637 12.3013) (width 0.25) (layer "F.Cu") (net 2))
 (segment (start 21.025 7.9894) (end 20.0686 7.033) (width 0.25) (layer "F.Cu") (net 2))
 (segment (start 10.8945 12.3013) (end 9.4176 10.8244) (width 0.25) (layer "F.Cu") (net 2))
 (segment (start 9.96 13.2358) (end 10.8945 12.3013) (width 0.25) (layer "F.Cu") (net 2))
 (segment (start 14.8505 4.7415) (end 14.8505 5.822) (width 0.25) (layer "F.Cu") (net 2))
 (segment (start 11.075 1.875) (end 11.8137 2.6137) (width 0.25) (layer "F.Cu") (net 2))
 (segment (start 14.1669 4.0579) (end 14.8505 4.7415) (width 0.25) (layer "F.Cu") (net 2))
 (segment (start 20.0686 7.033) (end 20.0686 2.9844) (width 0.25) (layer "F.Cu") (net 2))
 (segment (start 17.5142 6.2346) (end 17.5142 5.9611) (width 0.25) (layer "F.Cu") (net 2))
 (segment (start 21.025 8.225) (end 21.025 7.9894) (width 0.25) (layer "F.Cu") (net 2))
 (segment (start 20.0686 7.033) (end 18.3126 7.033) (width 0.25) (layer "F.Cu") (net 2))
 (segment (start 10.4423 6.7548) (end 11.55 7.8625) (width 0.25) (layer "F.Cu") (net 2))
 (segment (start 14.9845 5.822) (end 14.8505 5.822) (width 0.25) (layer "F.Cu") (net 2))
 (via (at 14.8505 5.822) (size 0.6) (drill 0.3) (layers "F.Cu" "B.Cu") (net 2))
 (via (at 10.4423 5.9042) (size 0.6) (drill 0.3) (layers "F.Cu" "B.Cu") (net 2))
 (segment (start 4.9733 16.8817) (end 2.5628 16.8817) (width 0.25) (layer "B.Cu") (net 2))
 (segment (start 2.4024 13.9441) (end 10.4423 5.9042) (width 0.25) (layer "B.Cu") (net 2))
 (segment (start 14.7683 5.9042) (end 14.8505 5.822) (width 0.25) (layer "B.Cu") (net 2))
 (segment (start 10.4423 5.9042) (end 14.7683 5.9042) (width 0.25) (layer "B.Cu") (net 2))
 (segment (start 2.4024 16.7213) (end 2.4024 13.9441) (width 0.25) (layer "B.Cu") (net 2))
 (segment (start 6.15 15.705) (end 4.9733 16.8817) (width 0.25) (layer "B.Cu") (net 2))
 (segment (start 2.5628 16.8817) (end 2.4024 16.7213) (width 0.25) (layer "B.Cu") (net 2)))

